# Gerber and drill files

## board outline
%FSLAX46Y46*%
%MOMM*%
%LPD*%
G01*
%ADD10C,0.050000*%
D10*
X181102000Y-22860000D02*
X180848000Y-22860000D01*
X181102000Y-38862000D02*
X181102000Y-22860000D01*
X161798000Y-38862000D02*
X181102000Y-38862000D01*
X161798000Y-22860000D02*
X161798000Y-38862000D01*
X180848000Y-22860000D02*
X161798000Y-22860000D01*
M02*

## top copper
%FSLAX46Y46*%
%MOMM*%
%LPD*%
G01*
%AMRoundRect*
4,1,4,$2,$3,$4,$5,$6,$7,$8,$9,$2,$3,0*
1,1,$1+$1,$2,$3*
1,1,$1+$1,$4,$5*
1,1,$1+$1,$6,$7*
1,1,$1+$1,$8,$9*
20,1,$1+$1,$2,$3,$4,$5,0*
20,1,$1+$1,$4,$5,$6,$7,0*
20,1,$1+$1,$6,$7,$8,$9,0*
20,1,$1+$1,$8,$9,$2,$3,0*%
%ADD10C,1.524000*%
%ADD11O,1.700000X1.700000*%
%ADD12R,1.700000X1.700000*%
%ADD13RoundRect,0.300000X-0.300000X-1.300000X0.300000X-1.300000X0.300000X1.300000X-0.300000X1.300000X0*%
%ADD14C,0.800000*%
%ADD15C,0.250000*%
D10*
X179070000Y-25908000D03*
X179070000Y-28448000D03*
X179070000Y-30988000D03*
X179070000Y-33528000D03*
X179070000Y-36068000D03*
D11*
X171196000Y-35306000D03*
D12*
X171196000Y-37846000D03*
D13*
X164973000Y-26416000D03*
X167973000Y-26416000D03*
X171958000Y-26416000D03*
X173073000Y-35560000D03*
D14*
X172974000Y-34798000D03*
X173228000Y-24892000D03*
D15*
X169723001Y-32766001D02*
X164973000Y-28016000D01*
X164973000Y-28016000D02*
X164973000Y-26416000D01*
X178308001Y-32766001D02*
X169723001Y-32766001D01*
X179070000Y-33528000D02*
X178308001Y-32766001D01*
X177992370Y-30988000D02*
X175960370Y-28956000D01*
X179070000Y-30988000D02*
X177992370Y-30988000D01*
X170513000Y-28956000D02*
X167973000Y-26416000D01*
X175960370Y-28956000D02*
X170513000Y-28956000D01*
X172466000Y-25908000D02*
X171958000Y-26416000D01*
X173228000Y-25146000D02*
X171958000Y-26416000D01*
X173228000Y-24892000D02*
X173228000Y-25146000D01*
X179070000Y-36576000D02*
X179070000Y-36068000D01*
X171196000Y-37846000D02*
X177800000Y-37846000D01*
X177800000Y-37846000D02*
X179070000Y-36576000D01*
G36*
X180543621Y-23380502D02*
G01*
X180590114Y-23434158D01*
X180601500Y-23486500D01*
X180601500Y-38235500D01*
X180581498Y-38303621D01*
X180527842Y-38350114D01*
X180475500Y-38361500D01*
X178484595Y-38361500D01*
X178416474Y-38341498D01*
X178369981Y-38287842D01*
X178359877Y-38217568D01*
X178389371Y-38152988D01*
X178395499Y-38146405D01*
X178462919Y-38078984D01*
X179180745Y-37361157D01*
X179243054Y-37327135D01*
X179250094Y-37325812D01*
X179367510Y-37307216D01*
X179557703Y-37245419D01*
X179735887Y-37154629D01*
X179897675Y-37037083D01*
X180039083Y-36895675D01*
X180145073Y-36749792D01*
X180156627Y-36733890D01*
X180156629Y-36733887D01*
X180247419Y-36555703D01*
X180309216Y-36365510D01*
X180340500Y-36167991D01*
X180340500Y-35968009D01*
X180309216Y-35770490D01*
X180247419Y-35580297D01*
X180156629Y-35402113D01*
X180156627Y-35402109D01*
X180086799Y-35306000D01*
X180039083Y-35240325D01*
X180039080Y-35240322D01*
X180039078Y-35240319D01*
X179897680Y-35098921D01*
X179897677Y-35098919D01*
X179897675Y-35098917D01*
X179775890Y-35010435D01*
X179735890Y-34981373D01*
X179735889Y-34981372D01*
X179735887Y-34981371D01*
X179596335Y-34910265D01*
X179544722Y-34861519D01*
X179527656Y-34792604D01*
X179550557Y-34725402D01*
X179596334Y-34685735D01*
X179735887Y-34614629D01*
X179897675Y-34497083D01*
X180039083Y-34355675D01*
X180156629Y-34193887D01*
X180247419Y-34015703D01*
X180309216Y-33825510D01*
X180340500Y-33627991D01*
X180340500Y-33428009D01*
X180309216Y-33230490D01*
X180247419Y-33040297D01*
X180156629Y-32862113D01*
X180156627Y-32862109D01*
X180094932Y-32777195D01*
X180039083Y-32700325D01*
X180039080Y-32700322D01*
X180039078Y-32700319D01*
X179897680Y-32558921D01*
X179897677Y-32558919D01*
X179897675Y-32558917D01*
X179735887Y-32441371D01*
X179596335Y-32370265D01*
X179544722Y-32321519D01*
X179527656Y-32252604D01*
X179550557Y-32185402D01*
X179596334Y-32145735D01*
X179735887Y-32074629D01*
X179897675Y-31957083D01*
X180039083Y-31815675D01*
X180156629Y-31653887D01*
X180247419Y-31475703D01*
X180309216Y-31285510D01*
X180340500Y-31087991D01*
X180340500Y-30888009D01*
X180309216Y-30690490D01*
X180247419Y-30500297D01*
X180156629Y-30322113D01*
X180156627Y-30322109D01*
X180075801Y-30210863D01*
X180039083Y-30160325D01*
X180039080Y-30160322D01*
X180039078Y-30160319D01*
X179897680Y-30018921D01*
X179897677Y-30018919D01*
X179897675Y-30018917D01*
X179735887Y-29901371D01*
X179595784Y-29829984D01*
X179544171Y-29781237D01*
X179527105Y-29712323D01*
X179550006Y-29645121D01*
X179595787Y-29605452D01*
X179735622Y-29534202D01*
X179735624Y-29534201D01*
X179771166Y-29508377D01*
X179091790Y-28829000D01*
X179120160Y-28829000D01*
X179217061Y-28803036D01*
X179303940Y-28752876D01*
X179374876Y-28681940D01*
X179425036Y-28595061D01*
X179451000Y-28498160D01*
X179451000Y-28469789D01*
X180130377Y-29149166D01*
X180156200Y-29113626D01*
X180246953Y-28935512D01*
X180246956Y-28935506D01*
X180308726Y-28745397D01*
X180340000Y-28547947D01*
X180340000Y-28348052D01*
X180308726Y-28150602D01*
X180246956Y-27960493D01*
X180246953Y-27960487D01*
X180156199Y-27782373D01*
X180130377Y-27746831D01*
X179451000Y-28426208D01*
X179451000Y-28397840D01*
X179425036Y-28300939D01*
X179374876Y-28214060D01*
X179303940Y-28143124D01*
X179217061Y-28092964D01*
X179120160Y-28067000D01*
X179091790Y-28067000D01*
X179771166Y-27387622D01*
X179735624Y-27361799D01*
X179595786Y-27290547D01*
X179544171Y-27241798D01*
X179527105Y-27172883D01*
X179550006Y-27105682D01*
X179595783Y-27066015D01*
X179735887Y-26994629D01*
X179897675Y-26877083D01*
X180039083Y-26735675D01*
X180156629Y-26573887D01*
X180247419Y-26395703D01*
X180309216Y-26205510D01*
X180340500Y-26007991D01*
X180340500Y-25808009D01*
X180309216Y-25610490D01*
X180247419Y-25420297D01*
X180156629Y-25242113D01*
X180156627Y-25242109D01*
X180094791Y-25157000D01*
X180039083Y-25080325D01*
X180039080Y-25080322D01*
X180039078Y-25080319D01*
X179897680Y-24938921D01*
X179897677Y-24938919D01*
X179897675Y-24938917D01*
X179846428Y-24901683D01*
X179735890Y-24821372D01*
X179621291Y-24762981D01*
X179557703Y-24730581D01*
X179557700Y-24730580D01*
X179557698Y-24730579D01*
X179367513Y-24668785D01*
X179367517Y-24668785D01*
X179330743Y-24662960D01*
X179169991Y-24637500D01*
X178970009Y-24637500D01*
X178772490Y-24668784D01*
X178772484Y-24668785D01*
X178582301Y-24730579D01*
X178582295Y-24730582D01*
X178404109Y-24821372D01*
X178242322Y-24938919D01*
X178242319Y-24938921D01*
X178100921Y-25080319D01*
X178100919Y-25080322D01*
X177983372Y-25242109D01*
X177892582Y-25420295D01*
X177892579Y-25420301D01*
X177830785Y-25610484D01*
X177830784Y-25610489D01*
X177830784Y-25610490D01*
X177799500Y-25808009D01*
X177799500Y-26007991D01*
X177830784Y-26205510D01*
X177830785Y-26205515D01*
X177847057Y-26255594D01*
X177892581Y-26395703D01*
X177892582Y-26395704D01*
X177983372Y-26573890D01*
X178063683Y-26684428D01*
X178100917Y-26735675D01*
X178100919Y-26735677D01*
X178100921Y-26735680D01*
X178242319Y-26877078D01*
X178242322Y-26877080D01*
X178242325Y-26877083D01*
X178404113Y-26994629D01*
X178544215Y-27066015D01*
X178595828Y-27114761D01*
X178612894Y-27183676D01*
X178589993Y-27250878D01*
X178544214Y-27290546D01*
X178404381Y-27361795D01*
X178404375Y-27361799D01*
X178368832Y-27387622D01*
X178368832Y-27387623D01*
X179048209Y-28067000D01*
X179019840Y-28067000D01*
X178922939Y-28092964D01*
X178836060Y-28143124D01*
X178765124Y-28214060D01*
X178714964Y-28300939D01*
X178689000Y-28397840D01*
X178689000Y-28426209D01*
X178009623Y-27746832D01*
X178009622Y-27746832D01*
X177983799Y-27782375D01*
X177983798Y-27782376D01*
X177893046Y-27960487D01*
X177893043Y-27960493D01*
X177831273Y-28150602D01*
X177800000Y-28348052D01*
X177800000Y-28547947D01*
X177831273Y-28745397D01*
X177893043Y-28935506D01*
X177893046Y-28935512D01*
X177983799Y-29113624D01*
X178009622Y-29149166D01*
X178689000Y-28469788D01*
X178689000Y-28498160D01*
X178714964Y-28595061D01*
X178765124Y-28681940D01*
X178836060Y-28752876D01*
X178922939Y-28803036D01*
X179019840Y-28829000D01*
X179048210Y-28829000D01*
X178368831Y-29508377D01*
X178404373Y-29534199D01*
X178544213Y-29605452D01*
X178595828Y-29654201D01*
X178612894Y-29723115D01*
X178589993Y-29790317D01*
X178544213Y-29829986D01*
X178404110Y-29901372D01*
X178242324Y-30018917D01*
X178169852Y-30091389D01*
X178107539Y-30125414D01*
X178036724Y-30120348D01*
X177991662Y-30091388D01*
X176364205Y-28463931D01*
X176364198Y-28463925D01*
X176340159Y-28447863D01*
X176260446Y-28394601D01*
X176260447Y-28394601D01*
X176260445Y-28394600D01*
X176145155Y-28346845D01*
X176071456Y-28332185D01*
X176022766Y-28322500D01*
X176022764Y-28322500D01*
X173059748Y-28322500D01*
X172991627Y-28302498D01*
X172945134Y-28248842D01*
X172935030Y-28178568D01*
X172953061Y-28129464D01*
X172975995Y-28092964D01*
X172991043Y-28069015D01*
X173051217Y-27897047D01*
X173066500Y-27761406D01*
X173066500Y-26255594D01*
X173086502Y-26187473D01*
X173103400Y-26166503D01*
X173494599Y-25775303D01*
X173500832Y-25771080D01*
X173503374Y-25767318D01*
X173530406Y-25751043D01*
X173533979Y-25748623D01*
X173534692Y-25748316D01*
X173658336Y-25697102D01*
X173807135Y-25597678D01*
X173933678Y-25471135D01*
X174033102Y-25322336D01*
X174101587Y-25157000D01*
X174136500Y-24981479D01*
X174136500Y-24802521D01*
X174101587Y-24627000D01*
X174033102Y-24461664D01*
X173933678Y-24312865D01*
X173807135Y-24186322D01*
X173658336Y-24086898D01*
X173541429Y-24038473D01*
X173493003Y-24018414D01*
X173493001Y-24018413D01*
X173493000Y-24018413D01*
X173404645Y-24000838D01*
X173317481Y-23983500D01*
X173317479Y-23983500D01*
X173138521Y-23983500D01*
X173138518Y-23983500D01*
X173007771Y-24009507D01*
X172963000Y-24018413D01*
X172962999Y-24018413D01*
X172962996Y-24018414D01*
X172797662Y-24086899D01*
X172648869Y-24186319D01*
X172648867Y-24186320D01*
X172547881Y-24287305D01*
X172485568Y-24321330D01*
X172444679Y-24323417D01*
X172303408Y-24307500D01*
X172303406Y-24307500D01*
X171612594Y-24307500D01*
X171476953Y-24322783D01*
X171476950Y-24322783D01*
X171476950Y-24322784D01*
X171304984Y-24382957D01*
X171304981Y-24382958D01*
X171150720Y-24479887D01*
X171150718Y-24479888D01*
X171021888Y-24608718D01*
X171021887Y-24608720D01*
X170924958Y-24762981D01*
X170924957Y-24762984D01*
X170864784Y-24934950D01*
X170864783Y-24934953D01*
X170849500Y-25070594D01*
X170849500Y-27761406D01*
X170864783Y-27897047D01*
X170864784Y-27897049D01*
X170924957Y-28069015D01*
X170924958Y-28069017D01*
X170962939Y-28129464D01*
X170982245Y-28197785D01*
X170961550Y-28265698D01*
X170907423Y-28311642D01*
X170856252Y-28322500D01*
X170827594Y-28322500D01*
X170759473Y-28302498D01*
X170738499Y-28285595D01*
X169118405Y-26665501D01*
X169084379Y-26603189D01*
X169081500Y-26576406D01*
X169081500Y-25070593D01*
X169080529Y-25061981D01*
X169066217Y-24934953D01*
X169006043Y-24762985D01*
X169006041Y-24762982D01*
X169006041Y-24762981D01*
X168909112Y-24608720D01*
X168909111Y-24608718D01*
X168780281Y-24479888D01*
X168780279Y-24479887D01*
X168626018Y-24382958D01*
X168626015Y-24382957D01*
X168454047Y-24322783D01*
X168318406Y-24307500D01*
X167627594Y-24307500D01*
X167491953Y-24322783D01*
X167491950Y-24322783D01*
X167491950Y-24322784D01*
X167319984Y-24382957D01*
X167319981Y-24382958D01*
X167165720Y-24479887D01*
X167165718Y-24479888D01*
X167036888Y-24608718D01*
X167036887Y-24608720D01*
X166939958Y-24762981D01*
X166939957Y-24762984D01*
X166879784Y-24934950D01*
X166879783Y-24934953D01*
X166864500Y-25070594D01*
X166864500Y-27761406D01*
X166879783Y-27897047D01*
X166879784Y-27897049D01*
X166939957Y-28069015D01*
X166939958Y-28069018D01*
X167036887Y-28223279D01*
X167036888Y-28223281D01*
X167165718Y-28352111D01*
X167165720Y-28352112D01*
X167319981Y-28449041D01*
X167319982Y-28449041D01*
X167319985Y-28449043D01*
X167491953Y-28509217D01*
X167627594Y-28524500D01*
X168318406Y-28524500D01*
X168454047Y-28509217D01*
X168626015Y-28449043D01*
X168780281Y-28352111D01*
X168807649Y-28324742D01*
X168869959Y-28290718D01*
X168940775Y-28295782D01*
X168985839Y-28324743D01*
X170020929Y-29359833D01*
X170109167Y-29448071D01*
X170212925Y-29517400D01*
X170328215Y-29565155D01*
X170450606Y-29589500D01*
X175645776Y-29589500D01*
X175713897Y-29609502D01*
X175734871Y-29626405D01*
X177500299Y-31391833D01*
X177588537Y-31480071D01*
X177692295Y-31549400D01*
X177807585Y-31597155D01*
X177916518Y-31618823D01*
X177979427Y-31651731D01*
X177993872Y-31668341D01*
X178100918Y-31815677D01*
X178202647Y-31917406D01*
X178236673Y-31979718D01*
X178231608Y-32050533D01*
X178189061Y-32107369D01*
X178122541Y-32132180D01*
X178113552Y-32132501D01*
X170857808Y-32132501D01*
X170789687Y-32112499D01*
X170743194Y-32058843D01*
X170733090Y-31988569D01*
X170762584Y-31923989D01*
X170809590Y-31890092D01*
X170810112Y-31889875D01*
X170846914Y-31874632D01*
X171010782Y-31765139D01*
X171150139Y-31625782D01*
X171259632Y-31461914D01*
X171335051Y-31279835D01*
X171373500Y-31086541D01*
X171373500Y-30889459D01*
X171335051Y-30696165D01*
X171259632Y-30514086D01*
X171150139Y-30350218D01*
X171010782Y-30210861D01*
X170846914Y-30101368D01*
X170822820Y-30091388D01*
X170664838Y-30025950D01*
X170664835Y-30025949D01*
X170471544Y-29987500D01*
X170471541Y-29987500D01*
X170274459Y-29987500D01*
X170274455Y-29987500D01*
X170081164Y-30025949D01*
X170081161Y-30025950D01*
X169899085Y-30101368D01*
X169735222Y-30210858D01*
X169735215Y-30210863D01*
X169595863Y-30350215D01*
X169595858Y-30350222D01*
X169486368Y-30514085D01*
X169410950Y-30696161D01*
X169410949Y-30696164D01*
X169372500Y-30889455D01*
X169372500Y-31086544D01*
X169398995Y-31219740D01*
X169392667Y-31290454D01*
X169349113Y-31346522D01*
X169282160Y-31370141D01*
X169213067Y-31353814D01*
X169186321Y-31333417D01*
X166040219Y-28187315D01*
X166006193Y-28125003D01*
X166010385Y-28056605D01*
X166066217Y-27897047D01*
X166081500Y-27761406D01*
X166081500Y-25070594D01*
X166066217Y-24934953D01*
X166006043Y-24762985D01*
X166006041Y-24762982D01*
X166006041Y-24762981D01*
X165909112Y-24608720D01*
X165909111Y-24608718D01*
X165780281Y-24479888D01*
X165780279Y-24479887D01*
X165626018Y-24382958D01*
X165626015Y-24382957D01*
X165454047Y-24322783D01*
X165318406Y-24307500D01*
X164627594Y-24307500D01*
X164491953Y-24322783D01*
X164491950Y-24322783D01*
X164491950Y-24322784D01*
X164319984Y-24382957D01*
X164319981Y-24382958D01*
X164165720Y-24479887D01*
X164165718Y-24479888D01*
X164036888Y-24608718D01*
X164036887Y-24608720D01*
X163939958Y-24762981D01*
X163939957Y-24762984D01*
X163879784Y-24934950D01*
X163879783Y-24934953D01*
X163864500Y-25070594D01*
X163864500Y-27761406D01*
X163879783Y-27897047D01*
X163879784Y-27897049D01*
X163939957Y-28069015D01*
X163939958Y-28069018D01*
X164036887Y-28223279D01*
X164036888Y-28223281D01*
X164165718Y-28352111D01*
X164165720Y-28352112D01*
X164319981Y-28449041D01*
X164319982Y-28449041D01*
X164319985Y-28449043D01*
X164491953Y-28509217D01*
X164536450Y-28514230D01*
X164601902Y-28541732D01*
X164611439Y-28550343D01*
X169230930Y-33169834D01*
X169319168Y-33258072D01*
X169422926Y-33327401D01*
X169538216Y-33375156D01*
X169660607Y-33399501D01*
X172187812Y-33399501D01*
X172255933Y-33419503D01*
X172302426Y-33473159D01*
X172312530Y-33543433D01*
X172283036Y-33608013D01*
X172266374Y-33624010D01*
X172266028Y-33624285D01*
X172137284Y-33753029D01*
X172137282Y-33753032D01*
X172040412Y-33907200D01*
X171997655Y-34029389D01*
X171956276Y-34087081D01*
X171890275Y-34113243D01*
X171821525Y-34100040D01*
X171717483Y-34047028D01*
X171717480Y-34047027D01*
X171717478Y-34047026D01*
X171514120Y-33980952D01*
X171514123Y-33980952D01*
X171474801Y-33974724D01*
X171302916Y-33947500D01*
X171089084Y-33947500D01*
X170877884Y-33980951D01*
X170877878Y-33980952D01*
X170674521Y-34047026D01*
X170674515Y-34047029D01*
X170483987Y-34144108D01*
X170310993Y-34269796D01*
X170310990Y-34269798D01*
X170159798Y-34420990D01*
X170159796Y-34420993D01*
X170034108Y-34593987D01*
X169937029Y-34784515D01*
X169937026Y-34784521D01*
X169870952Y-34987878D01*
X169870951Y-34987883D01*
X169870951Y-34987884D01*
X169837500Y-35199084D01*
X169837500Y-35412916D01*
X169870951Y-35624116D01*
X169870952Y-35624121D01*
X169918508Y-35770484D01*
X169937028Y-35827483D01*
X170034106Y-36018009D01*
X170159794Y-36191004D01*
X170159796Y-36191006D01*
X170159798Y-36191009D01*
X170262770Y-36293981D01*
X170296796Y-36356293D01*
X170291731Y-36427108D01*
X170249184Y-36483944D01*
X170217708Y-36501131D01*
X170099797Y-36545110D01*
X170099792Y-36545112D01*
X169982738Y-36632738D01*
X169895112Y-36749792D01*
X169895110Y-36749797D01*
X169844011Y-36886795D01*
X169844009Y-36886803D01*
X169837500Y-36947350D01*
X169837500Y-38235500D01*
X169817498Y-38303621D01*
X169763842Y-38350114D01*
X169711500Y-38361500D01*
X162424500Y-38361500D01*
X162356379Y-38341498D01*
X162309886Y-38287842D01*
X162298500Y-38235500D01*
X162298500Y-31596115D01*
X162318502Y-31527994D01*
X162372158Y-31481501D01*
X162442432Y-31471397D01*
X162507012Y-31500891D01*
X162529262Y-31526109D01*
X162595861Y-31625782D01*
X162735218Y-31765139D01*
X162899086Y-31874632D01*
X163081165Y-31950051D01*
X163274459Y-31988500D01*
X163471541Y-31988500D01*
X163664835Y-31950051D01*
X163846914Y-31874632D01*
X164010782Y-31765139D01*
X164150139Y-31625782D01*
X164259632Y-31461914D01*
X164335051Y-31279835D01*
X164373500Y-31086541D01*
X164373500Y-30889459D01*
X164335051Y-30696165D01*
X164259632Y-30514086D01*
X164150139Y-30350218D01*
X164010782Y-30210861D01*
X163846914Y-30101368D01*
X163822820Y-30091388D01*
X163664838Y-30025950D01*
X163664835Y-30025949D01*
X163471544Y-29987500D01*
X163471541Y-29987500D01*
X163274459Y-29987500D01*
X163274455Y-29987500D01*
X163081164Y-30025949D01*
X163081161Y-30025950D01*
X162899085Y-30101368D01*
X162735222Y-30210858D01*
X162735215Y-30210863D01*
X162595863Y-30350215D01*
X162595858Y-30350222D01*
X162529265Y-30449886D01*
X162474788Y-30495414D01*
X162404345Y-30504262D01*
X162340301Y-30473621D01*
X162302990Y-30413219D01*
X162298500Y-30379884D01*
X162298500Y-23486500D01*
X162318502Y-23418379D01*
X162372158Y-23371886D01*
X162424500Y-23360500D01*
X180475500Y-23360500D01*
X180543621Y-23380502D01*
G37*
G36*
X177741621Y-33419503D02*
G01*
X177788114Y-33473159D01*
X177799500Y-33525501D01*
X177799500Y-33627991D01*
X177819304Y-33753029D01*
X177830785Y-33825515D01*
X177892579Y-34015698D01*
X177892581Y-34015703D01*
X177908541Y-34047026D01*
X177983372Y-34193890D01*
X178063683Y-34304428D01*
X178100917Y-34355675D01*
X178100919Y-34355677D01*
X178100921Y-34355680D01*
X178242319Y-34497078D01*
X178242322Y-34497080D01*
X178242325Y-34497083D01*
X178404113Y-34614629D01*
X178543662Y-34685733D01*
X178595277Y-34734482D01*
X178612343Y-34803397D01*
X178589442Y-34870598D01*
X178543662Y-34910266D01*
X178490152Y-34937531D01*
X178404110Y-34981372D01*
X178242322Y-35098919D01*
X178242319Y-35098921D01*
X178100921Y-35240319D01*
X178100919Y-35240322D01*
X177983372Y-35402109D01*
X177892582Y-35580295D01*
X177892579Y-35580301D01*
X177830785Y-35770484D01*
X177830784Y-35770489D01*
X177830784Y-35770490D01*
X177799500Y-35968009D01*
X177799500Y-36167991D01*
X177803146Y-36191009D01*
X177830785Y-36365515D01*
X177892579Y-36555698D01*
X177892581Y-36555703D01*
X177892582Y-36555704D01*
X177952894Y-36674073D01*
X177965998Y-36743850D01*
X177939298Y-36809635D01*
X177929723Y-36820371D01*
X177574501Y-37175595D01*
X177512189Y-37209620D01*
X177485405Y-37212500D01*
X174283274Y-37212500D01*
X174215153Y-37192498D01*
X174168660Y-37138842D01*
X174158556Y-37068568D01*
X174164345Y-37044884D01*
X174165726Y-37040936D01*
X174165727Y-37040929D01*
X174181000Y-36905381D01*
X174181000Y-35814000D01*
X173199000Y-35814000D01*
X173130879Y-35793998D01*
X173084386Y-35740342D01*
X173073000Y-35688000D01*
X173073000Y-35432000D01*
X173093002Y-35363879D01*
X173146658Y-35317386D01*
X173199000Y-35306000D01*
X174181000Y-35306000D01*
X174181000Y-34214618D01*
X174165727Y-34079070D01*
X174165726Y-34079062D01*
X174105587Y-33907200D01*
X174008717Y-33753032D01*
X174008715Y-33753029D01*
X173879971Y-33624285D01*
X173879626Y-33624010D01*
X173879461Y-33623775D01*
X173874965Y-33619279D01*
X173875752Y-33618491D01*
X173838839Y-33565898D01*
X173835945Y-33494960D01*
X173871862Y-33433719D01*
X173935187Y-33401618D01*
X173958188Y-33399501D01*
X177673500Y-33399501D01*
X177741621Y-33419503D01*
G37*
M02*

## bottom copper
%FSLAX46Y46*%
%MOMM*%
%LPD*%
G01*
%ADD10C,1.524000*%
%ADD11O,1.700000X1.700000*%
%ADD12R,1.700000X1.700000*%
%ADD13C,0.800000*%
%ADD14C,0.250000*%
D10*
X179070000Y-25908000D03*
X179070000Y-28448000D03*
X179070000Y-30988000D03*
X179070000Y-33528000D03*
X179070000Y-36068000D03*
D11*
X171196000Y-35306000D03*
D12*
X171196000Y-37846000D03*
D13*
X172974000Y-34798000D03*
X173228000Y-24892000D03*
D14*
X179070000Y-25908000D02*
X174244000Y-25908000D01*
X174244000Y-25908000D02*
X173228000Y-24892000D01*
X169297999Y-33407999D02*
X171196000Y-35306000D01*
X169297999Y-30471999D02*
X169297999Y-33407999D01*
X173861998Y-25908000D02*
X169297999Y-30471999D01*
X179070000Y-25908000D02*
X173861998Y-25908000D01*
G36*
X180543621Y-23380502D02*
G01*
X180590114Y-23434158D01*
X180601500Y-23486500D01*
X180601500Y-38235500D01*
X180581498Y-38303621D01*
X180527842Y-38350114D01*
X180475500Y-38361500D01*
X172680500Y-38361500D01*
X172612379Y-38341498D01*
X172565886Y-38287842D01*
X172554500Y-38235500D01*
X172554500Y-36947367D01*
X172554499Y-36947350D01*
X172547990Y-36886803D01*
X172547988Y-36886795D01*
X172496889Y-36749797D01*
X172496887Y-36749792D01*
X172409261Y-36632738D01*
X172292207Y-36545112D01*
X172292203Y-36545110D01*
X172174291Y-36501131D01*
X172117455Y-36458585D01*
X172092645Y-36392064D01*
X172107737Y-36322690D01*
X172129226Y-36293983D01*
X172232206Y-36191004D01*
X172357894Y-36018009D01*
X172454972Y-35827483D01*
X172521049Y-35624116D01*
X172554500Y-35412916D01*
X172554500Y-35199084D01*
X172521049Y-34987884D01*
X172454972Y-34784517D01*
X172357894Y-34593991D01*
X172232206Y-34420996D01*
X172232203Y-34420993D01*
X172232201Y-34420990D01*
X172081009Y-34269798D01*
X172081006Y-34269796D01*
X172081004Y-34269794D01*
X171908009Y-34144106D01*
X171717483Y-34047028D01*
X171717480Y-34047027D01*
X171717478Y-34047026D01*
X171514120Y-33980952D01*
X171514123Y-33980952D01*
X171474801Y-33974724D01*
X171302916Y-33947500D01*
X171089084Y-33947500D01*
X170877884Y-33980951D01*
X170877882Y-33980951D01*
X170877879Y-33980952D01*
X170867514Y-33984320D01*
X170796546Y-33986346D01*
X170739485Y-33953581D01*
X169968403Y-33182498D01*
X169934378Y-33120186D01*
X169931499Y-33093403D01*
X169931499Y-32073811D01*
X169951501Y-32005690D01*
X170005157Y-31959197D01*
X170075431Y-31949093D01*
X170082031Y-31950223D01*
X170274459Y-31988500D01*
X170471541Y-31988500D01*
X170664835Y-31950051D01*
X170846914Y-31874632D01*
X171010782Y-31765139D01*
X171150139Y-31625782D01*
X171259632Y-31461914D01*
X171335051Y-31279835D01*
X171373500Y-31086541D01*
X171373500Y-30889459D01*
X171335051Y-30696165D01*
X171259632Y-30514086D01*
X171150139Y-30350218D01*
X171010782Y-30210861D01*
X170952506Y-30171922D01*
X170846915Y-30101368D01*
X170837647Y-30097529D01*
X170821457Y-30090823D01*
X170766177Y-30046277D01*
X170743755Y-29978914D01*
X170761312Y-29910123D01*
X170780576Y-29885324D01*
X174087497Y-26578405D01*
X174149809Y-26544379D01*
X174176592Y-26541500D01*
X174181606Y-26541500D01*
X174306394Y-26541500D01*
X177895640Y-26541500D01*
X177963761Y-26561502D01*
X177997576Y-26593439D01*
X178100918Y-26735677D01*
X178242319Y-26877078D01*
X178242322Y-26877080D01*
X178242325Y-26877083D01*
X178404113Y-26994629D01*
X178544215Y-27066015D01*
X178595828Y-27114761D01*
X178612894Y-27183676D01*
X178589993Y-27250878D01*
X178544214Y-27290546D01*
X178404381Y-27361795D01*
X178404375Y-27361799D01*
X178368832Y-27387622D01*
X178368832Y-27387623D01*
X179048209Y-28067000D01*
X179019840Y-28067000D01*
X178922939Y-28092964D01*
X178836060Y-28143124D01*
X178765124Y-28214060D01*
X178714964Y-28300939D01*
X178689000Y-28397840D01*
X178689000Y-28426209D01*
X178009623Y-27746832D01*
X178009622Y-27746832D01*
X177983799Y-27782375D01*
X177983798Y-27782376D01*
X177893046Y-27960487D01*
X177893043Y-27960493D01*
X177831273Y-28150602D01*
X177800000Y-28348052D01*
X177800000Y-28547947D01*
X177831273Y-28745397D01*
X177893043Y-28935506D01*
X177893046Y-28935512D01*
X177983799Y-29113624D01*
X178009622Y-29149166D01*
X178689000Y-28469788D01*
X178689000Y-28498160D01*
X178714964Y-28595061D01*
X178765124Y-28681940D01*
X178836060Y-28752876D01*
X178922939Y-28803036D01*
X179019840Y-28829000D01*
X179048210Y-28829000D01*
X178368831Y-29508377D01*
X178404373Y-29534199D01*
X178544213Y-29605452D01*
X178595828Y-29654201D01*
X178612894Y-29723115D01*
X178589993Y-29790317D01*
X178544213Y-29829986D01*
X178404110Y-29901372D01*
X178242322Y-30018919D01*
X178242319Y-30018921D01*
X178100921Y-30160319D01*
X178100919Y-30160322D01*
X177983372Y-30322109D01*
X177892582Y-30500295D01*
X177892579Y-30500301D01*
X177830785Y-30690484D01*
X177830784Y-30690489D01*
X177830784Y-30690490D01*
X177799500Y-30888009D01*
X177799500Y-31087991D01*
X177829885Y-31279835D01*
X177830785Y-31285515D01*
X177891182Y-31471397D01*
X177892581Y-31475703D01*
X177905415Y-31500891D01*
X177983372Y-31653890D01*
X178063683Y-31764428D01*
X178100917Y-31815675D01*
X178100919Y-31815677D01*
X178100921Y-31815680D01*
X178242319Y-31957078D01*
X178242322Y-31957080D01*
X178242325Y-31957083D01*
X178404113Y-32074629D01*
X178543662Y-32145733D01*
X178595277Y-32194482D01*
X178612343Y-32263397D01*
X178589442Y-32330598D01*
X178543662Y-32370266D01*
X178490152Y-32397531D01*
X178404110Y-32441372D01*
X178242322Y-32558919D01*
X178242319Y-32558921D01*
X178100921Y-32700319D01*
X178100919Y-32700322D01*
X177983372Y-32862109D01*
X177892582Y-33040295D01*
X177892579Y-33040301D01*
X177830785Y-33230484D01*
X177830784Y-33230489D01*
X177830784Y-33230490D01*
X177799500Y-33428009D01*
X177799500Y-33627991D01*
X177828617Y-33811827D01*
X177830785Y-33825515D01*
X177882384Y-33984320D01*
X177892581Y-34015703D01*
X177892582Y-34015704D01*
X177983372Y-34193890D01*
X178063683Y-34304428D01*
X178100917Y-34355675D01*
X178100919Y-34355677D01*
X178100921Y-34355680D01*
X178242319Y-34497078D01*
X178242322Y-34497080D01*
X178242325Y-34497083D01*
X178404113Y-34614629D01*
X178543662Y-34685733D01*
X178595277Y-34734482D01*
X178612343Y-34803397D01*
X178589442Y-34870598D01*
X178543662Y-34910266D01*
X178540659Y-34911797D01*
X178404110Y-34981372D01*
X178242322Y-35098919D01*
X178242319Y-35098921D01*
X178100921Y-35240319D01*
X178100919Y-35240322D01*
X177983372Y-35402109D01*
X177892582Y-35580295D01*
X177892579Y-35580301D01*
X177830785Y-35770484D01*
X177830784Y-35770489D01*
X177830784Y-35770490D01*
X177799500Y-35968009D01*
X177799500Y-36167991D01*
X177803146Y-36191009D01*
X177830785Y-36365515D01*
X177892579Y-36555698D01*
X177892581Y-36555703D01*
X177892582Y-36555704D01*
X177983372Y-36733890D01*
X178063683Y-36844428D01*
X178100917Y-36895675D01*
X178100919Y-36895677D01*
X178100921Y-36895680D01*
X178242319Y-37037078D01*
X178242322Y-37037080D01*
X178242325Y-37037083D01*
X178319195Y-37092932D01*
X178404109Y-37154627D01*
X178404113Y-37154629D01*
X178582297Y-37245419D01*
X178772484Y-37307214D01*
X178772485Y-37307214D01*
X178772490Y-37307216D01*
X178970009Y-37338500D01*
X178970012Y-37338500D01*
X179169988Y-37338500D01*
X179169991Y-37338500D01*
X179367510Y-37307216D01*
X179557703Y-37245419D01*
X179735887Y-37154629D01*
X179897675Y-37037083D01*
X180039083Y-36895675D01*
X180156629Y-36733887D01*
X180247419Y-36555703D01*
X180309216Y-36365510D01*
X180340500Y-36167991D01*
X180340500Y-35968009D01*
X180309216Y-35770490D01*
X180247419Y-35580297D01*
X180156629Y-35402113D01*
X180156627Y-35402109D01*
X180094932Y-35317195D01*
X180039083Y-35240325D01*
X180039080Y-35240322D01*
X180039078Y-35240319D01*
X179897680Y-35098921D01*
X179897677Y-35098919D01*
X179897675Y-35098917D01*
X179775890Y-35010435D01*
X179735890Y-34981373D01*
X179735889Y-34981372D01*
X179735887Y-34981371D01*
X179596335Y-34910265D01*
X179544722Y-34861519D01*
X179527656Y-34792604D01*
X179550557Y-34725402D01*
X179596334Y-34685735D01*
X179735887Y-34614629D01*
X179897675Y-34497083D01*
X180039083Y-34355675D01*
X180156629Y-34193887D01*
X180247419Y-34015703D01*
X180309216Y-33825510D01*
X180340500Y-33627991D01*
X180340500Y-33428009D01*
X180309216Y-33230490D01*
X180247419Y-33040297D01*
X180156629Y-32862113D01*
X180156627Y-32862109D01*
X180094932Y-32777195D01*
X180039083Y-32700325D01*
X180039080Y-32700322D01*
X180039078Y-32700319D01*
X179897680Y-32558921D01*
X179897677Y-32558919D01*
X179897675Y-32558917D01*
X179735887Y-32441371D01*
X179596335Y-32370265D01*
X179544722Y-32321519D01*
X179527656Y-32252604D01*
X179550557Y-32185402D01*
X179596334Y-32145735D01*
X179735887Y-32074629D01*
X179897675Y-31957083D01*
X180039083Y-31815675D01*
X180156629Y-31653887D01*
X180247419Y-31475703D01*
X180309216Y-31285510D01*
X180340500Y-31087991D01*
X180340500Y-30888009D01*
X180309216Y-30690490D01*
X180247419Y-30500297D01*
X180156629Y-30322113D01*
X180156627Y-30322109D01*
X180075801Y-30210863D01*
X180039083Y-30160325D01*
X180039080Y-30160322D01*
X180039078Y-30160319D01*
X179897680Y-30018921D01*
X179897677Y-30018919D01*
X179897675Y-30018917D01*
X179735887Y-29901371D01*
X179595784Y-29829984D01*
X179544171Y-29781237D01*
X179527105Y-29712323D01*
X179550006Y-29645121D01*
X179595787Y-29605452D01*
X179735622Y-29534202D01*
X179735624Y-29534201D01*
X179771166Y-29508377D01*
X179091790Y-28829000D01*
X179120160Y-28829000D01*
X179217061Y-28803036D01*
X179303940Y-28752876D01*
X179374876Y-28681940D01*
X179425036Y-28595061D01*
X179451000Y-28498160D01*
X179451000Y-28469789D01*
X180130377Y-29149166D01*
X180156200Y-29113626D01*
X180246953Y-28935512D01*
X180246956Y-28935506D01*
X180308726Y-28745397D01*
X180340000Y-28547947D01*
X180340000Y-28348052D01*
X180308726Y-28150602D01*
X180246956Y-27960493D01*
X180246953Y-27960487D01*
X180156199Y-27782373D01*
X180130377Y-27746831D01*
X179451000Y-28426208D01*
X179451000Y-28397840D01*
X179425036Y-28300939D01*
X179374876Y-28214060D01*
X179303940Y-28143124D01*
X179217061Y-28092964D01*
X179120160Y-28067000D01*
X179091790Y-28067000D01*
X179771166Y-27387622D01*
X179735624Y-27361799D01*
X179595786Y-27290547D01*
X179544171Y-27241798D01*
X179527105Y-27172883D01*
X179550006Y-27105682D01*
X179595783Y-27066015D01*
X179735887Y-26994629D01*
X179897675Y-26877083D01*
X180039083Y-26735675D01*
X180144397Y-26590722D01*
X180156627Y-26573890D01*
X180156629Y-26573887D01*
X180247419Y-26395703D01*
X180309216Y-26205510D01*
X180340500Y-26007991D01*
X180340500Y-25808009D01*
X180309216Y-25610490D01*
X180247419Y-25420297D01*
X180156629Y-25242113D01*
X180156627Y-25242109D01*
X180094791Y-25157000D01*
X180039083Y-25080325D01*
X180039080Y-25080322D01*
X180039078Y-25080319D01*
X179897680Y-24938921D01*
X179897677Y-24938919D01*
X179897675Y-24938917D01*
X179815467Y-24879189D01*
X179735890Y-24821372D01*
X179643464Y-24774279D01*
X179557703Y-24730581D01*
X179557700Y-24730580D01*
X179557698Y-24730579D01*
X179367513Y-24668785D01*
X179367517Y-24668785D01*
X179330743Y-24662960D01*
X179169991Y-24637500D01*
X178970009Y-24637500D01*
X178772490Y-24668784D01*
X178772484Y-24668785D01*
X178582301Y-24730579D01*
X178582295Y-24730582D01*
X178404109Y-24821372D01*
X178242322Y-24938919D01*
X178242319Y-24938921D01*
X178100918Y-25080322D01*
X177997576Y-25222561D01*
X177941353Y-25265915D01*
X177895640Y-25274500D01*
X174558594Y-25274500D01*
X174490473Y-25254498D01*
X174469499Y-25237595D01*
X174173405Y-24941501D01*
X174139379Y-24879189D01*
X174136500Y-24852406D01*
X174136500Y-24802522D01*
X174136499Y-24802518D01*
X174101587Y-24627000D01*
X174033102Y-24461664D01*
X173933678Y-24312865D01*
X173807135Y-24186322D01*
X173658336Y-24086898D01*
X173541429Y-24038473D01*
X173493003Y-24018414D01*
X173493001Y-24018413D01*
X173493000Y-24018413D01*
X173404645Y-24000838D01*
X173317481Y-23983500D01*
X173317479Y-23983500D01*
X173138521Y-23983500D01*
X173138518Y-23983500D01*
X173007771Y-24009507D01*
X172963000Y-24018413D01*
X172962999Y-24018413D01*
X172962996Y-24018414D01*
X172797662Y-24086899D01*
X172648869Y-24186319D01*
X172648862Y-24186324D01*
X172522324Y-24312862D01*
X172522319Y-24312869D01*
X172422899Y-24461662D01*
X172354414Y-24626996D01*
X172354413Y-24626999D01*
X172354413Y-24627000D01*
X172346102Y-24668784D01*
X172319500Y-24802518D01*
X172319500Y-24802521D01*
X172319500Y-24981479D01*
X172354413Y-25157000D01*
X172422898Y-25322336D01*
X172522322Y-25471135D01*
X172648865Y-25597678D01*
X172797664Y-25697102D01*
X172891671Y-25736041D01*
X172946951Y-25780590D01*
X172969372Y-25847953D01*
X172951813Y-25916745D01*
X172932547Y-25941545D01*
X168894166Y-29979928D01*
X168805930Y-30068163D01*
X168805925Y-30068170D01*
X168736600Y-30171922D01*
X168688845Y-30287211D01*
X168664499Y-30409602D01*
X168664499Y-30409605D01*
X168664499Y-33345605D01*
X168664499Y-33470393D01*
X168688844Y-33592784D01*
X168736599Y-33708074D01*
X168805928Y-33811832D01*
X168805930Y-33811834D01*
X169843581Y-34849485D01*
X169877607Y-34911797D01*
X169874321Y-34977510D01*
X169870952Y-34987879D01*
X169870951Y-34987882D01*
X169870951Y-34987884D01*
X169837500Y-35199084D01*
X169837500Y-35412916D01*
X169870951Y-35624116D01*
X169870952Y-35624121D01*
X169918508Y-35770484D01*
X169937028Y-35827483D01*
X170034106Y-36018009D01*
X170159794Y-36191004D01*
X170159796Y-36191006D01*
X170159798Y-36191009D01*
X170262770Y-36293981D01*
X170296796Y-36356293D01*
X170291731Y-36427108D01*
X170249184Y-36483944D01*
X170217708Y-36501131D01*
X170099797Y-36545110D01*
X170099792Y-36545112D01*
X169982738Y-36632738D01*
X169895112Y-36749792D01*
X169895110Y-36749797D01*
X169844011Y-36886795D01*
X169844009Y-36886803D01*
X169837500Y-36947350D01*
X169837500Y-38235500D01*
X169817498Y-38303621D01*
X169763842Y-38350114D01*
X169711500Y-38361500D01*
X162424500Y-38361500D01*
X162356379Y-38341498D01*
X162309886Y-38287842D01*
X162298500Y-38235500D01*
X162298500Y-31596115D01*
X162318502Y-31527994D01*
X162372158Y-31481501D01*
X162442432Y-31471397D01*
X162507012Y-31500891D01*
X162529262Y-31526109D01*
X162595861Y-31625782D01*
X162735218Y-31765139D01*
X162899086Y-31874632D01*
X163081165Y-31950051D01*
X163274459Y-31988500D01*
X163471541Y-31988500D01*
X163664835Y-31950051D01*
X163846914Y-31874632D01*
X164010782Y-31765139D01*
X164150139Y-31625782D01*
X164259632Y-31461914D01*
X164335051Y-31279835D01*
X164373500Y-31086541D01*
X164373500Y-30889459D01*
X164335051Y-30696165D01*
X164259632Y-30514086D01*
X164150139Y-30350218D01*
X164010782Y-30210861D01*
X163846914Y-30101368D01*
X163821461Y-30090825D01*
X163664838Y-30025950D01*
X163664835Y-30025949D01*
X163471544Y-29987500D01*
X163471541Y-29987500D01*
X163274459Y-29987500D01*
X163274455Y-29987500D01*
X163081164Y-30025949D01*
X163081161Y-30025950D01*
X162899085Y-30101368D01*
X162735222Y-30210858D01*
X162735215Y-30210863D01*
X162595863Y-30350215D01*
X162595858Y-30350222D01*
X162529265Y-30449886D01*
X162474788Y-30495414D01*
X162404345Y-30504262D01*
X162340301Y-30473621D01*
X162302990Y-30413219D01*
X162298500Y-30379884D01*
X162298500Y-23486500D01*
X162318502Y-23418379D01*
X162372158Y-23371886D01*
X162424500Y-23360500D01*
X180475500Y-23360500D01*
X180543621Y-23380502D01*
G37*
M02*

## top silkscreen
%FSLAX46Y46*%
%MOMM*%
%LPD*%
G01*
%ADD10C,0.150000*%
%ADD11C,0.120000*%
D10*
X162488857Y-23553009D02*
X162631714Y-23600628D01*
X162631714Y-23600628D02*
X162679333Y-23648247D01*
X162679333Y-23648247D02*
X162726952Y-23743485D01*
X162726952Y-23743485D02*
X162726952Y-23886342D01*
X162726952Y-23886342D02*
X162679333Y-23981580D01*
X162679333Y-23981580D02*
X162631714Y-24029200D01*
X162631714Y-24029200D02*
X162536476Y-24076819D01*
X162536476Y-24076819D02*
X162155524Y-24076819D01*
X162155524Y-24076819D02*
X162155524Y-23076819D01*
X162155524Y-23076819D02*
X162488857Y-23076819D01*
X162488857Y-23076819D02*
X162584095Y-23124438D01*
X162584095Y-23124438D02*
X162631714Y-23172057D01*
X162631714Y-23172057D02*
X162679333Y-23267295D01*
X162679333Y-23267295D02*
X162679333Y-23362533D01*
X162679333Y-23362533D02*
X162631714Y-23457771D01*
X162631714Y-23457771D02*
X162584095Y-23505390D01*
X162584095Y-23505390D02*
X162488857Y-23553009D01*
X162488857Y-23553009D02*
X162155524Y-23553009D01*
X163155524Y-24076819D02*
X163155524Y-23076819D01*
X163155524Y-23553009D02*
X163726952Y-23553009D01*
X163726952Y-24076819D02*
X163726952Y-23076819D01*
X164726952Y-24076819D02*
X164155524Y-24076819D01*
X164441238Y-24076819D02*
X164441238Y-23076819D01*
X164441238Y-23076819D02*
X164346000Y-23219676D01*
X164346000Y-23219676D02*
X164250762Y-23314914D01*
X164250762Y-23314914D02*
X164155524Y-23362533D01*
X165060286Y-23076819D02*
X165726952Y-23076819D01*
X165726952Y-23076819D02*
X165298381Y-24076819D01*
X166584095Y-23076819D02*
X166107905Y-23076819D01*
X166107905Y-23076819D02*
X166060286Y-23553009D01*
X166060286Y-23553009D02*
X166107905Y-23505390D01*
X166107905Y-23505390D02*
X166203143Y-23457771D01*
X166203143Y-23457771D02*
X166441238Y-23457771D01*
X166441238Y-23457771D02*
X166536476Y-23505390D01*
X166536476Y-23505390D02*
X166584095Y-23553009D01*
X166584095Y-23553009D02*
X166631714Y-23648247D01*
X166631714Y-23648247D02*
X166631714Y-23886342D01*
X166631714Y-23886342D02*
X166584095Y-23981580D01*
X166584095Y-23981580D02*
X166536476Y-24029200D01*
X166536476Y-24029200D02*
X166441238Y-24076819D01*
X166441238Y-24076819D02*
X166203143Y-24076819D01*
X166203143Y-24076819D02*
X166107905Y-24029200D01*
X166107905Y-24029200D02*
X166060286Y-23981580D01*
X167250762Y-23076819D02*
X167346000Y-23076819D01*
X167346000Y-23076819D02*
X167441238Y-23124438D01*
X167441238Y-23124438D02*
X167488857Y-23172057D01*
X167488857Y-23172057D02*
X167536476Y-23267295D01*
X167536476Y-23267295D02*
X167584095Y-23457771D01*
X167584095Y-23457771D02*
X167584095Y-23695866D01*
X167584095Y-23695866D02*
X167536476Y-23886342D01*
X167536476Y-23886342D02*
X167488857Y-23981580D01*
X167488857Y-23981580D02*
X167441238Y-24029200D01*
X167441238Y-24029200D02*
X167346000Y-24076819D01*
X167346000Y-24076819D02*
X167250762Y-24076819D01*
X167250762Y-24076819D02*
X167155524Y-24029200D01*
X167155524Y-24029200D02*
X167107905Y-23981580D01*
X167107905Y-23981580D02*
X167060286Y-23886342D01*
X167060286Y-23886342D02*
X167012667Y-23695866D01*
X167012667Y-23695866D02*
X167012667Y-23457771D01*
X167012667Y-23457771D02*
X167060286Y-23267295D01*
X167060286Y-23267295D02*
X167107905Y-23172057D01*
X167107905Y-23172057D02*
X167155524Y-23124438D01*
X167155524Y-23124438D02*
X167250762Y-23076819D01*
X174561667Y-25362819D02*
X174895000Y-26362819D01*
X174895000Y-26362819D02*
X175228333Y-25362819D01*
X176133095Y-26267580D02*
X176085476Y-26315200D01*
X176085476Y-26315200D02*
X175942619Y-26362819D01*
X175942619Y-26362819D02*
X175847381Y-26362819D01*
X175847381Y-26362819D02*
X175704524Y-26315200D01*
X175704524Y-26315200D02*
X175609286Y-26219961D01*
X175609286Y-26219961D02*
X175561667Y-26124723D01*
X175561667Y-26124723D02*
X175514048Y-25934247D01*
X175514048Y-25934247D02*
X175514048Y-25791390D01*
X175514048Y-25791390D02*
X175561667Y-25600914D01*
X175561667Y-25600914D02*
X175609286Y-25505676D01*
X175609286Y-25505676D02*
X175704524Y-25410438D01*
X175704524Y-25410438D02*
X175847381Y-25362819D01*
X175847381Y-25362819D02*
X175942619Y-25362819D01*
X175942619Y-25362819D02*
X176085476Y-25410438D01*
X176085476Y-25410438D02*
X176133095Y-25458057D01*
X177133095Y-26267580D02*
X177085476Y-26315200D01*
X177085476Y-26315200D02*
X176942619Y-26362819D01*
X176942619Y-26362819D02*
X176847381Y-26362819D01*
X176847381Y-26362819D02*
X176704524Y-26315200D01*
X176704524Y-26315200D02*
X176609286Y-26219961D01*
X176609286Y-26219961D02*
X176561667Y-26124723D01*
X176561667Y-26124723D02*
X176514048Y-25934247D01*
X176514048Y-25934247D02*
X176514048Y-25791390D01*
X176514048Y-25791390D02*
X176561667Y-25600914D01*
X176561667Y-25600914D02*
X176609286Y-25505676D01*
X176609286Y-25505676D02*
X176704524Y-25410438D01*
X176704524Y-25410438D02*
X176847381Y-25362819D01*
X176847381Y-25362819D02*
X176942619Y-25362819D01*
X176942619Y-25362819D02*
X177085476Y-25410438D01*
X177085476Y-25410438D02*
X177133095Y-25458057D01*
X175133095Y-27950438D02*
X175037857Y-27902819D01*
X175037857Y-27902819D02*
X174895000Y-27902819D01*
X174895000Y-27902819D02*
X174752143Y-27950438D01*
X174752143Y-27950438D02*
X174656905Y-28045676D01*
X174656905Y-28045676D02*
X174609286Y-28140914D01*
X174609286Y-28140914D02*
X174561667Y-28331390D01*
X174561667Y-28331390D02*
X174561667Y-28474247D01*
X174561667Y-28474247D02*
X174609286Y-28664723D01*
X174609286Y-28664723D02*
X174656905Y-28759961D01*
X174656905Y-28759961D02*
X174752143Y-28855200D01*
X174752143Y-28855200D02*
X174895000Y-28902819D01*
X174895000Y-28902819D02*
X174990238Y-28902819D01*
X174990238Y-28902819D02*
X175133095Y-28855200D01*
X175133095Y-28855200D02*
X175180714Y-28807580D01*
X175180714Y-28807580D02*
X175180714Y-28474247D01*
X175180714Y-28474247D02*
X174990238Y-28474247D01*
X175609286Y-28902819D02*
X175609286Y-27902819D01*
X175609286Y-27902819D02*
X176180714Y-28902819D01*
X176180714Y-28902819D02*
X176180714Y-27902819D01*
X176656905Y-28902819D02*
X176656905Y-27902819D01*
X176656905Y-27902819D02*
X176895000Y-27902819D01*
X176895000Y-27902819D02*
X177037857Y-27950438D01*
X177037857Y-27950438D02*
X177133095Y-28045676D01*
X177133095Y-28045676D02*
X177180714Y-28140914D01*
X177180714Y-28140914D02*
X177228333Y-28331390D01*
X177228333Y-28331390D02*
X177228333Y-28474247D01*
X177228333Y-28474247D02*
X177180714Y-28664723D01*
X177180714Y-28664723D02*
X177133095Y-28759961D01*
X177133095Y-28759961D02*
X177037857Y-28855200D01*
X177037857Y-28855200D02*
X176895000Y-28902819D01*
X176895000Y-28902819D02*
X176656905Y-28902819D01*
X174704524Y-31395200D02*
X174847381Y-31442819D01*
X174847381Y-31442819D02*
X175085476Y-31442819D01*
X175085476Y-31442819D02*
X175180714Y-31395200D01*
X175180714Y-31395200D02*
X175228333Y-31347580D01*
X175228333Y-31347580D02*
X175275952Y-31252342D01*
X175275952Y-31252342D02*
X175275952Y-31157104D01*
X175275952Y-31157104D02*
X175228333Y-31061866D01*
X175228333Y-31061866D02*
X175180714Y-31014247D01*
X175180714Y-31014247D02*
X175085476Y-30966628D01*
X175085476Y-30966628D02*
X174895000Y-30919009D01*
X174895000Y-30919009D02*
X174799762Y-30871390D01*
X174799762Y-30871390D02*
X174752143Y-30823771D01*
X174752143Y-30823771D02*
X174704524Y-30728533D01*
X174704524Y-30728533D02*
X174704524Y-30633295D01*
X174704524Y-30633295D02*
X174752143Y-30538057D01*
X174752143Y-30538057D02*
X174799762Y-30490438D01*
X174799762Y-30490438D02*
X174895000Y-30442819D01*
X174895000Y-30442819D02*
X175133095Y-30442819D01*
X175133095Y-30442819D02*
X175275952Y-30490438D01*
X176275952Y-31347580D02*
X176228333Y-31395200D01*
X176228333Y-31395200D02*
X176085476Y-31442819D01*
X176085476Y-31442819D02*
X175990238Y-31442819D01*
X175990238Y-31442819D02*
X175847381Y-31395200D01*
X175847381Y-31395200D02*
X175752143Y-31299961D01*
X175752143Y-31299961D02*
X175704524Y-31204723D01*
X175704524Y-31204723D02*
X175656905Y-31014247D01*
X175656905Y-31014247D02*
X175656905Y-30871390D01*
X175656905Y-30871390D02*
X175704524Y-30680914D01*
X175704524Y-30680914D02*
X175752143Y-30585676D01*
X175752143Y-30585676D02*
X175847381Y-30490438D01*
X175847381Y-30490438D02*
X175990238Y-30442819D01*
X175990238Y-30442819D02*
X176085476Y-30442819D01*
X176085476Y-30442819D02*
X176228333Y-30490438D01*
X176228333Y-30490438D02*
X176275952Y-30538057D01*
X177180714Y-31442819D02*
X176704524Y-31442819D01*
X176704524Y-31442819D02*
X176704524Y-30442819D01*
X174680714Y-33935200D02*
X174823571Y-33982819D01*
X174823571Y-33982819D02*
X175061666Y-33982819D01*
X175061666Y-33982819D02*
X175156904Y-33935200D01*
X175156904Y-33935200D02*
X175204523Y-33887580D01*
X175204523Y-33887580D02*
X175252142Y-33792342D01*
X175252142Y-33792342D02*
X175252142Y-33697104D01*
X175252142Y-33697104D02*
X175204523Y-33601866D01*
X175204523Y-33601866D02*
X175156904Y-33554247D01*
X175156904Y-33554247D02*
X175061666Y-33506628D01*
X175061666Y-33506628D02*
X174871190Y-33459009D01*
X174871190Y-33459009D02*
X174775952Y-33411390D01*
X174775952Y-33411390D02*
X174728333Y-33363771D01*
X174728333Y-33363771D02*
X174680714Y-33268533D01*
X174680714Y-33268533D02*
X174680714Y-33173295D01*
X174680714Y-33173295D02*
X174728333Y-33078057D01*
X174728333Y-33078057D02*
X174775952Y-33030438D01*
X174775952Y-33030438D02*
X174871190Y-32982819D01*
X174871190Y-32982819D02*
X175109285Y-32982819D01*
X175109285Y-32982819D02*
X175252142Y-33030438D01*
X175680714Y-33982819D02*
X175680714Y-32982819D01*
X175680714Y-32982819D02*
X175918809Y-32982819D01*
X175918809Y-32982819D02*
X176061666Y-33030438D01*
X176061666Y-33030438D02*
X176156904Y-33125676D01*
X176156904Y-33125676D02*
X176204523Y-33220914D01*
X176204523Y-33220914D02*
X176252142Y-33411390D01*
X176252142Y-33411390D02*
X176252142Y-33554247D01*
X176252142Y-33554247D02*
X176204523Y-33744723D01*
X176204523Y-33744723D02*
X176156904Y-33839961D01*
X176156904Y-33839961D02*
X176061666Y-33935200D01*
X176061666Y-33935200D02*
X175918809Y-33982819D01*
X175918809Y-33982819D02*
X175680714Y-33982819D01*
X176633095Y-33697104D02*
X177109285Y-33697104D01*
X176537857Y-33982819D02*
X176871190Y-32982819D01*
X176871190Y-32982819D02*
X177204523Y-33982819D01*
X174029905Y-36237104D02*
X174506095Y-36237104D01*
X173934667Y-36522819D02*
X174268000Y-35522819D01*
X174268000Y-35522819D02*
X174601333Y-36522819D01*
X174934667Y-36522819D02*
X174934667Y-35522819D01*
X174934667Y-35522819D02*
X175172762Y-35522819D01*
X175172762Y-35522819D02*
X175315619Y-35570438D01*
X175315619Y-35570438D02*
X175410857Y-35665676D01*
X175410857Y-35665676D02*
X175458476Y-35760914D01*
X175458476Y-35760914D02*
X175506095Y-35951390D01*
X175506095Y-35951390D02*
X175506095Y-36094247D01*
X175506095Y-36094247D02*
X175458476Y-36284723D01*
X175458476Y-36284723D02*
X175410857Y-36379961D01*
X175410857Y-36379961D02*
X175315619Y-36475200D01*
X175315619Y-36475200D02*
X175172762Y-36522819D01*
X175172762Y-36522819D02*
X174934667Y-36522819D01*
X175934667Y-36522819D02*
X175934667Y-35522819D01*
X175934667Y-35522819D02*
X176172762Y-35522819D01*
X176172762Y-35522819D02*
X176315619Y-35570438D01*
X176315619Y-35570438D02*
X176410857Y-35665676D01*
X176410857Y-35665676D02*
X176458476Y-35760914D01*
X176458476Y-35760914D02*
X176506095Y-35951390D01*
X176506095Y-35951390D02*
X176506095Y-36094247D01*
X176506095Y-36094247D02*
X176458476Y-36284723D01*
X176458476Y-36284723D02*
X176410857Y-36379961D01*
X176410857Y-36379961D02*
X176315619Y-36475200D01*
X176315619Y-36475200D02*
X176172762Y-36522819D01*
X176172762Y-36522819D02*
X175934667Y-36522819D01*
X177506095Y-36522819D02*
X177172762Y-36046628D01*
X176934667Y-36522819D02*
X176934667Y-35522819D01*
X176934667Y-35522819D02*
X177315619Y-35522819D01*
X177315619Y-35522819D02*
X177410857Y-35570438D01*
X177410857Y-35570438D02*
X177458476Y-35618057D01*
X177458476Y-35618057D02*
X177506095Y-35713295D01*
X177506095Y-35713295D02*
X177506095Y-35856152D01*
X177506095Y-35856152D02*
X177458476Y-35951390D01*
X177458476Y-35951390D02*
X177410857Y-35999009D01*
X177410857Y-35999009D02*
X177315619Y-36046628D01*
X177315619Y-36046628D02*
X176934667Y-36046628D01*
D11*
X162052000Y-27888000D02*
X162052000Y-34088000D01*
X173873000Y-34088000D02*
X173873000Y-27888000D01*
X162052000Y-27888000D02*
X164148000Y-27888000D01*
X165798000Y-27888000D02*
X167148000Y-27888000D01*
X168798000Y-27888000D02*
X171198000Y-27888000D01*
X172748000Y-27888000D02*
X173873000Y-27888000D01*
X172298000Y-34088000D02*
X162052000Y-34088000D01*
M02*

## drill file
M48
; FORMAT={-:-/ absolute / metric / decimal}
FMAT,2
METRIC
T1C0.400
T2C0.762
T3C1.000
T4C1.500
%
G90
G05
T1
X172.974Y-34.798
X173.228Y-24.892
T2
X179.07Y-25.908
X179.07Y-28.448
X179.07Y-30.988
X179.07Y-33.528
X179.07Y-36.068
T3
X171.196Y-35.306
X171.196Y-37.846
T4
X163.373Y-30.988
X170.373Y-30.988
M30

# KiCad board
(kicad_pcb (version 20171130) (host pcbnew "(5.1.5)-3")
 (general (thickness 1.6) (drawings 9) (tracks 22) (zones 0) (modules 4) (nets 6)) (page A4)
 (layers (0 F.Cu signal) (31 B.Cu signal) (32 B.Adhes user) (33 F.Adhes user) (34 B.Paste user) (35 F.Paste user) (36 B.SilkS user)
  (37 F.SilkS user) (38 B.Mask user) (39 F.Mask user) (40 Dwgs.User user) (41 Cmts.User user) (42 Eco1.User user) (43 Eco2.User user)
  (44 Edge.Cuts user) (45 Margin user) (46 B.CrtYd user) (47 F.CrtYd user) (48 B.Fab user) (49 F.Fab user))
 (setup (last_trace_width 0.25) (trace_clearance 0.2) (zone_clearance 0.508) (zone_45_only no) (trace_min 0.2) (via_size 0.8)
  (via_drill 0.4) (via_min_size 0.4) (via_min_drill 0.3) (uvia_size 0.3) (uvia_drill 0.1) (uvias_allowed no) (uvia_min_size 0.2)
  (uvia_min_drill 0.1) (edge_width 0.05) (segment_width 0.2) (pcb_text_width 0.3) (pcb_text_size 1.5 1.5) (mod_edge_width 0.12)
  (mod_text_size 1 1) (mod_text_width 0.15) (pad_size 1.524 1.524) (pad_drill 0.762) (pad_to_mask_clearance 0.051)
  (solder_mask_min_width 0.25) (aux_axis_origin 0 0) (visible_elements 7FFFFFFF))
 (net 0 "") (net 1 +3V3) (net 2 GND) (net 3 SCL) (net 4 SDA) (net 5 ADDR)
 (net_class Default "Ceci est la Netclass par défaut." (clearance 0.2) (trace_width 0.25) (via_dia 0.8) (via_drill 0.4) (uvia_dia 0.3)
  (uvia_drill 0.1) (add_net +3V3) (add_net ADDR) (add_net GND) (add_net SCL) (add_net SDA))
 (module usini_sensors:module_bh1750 (layer F.Cu) (at 179.07 25.908 180)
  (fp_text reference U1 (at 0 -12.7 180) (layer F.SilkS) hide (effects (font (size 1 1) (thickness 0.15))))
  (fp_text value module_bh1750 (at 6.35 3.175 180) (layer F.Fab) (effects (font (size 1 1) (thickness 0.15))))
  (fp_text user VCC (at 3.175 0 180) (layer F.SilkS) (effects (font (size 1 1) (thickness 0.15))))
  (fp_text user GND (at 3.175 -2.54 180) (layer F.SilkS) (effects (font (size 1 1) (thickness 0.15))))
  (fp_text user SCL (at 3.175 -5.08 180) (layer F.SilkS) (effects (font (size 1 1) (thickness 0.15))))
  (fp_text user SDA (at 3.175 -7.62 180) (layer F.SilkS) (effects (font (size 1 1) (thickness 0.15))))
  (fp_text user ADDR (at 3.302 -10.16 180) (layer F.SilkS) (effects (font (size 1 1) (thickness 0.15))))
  (pad 5 thru_hole circle (at 0 0 180) (size 1.524 1.524) (drill 0.762) (layers *.Cu *.Mask) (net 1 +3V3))
  (pad 4 thru_hole circle (at 0 -2.54 180) (size 1.524 1.524) (drill 0.762) (layers *.Cu *.Mask) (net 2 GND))
  (pad 3 thru_hole circle (at 0 -5.08 180) (size 1.524 1.524) (drill 0.762) (layers *.Cu *.Mask) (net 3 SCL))
  (pad 2 thru_hole circle (at 0 -7.62 180) (size 1.524 1.524) (drill 0.762) (layers *.Cu *.Mask) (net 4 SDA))
  (pad 1 thru_hole circle (at 0 -10.16 180) (size 1.524 1.524) (drill 0.762) (layers *.Cu *.Mask) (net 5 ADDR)))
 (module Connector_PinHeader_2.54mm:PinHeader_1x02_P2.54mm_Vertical (layer F.Cu) (at 171.196 37.846 180)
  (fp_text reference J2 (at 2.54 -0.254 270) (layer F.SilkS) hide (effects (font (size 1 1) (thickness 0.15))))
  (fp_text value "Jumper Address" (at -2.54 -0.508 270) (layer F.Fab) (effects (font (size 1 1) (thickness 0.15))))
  (pad 2 thru_hole oval (at 0 2.54 180) (size 1.7 1.7) (drill 1) (layers *.Cu *.Mask) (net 1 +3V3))
  (pad 1 thru_hole rect (at 0 0 180) (size 1.7 1.7) (drill 1) (layers *.Cu *.Mask) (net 5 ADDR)))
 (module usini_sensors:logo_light (layer B.Cu) (at 174.244 27.94)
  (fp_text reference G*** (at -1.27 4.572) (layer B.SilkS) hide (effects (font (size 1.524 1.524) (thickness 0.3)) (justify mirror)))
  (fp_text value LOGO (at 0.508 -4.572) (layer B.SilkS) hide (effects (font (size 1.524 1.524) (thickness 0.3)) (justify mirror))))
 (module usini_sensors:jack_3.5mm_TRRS (layer F.Cu) (at 168.148 30.988)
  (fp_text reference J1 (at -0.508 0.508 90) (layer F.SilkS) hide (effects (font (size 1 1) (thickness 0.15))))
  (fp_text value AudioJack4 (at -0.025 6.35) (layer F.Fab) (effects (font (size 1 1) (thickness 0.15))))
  (fp_line (start -6.096 -3.1) (end -6.096 3.1) (layer F.SilkS) (width 0.12))
  (fp_line (start 5.725 3.1) (end 5.725 -3.1) (layer F.SilkS) (width 0.12))
  (fp_line (start -6.096 -3.1) (end -4 -3.1) (layer F.SilkS) (width 0.12))
  (fp_line (start -2.35 -3.1) (end -1 -3.1) (layer F.SilkS) (width 0.12))
  (fp_line (start 0.65 -3.1) (end 3.05 -3.1) (layer F.SilkS) (width 0.12))
  (fp_line (start 4.6 -3.1) (end 5.725 -3.1) (layer F.SilkS) (width 0.12))
  (fp_line (start 4.15 3.1) (end -6.096 3.1) (layer F.SilkS) (width 0.12))
  (pad "" np_thru_hole circle (at 2.225 0) (size 1.5 1.5) (drill 1.5) (layers *.Cu *.Mask))
  (pad "" np_thru_hole circle (at -4.775 0) (size 1.5 1.5) (drill 1.5) (layers *.Cu *.Mask))
  (pad R2 smd roundrect (at -3.175 -4.572) (size 1.2 3.2) (layers F.Cu F.Paste F.Mask) (roundrect_rratio 0.25) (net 4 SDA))
  (pad R1 smd roundrect (at -0.175 -4.572) (size 1.2 3.2) (layers F.Cu F.Paste F.Mask) (roundrect_rratio 0.25) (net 3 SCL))
  (pad T smd roundrect (at 3.81 -4.572) (size 1.2 3.2) (layers F.Cu F.Paste F.Mask) (roundrect_rratio 0.25) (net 1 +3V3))
  (pad S smd roundrect (at 4.925 4.572) (size 1.2 3.2) (layers F.Cu F.Paste F.Mask) (roundrect_rratio 0.25) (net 2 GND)))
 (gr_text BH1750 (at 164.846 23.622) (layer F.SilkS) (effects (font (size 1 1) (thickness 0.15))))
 (gr_line (start 181.102 22.86) (end 180.848 22.86) (layer Edge.Cuts) (width 0.05))
 (gr_line (start 181.102 38.862) (end 181.102 22.86) (layer Edge.Cuts) (width 0.05))
 (gr_line (start 161.798 38.862) (end 181.102 38.862) (layer Edge.Cuts) (width 0.05))
 (gr_line (start 161.798 22.86) (end 161.798 38.862) (layer Edge.Cuts) (width 0.05))
 (gr_line (start 180.848 22.86) (end 161.798 22.86) (layer Edge.Cuts) (width 0.05))
 (via (at 172.974 34.798) (size 0.8) (drill 0.4) (layers F.Cu B.Cu) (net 2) (status 30))
 (segment (start 169.723001 32.766001) (end 164.973 28.016) (width 0.25) (layer F.Cu) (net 4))
 (segment (start 164.973 28.016) (end 164.973 26.416) (width 0.25) (layer F.Cu) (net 4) (status 20))
 (segment (start 178.308001 32.766001) (end 169.723001 32.766001) (width 0.25) (layer F.Cu) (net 4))
 (segment (start 179.07 33.528) (end 178.308001 32.766001) (width 0.25) (layer F.Cu) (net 4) (status 10))
 (segment (start 177.99237 30.988) (end 175.96037 28.956) (width 0.25) (layer F.Cu) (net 3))
 (segment (start 179.07 30.988) (end 177.99237 30.988) (width 0.25) (layer F.Cu) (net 3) (status 10))
 (segment (start 170.513 28.956) (end 167.973 26.416) (width 0.25) (layer F.Cu) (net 3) (status 20))
 (segment (start 175.96037 28.956) (end 170.513 28.956) (width 0.25) (layer F.Cu) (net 3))
 (segment (start 172.466 25.908) (end 171.958 26.416) (width 0.25) (layer F.Cu) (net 1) (status 30))
 (via (at 173.228 24.892) (size 0.8) (drill 0.4) (layers F.Cu B.Cu) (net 1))
 (segment (start 179.07 25.908) (end 174.244 25.908) (width 0.25) (layer B.Cu) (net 1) (status 10))
 (segment (start 174.244 25.908) (end 173.228 24.892) (width 0.25) (layer B.Cu) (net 1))
 (segment (start 173.228 25.146) (end 171.958 26.416) (width 0.25) (layer F.Cu) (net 1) (status 20))
 (segment (start 173.228 24.892) (end 173.228 25.146) (width 0.25) (layer F.Cu) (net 1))
 (segment (start 169.297999 33.407999) (end 171.196 35.306) (width 0.25) (layer B.Cu) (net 1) (status 20))
 (segment (start 169.297999 30.471999) (end 169.297999 33.407999) (width 0.25) (layer B.Cu) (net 1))
 (segment (start 173.861998 25.908) (end 169.297999 30.471999) (width 0.25) (layer B.Cu) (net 1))
 (segment (start 179.07 25.908) (end 173.861998 25.908) (width 0.25) (layer B.Cu) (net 1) (status 10))
 (segment (start 179.07 36.576) (end 179.07 36.068) (width 0.25) (layer F.Cu) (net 5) (status 30))
 (segment (start 171.196 37.846) (end 177.8 37.846) (width 0.25) (layer F.Cu) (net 5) (status 10))
 (segment (start 177.8 37.846) (end 179.07 36.576) (width 0.25) (layer F.Cu) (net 5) (status 20))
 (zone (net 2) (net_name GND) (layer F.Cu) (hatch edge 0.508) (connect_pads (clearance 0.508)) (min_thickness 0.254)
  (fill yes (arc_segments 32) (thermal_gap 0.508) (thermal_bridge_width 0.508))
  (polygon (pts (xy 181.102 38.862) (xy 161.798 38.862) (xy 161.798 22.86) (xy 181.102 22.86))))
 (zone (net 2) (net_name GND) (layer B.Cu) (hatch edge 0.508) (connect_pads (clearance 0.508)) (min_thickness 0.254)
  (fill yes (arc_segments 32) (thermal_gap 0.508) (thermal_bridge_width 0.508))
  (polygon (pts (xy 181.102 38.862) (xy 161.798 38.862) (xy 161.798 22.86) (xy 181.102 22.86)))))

